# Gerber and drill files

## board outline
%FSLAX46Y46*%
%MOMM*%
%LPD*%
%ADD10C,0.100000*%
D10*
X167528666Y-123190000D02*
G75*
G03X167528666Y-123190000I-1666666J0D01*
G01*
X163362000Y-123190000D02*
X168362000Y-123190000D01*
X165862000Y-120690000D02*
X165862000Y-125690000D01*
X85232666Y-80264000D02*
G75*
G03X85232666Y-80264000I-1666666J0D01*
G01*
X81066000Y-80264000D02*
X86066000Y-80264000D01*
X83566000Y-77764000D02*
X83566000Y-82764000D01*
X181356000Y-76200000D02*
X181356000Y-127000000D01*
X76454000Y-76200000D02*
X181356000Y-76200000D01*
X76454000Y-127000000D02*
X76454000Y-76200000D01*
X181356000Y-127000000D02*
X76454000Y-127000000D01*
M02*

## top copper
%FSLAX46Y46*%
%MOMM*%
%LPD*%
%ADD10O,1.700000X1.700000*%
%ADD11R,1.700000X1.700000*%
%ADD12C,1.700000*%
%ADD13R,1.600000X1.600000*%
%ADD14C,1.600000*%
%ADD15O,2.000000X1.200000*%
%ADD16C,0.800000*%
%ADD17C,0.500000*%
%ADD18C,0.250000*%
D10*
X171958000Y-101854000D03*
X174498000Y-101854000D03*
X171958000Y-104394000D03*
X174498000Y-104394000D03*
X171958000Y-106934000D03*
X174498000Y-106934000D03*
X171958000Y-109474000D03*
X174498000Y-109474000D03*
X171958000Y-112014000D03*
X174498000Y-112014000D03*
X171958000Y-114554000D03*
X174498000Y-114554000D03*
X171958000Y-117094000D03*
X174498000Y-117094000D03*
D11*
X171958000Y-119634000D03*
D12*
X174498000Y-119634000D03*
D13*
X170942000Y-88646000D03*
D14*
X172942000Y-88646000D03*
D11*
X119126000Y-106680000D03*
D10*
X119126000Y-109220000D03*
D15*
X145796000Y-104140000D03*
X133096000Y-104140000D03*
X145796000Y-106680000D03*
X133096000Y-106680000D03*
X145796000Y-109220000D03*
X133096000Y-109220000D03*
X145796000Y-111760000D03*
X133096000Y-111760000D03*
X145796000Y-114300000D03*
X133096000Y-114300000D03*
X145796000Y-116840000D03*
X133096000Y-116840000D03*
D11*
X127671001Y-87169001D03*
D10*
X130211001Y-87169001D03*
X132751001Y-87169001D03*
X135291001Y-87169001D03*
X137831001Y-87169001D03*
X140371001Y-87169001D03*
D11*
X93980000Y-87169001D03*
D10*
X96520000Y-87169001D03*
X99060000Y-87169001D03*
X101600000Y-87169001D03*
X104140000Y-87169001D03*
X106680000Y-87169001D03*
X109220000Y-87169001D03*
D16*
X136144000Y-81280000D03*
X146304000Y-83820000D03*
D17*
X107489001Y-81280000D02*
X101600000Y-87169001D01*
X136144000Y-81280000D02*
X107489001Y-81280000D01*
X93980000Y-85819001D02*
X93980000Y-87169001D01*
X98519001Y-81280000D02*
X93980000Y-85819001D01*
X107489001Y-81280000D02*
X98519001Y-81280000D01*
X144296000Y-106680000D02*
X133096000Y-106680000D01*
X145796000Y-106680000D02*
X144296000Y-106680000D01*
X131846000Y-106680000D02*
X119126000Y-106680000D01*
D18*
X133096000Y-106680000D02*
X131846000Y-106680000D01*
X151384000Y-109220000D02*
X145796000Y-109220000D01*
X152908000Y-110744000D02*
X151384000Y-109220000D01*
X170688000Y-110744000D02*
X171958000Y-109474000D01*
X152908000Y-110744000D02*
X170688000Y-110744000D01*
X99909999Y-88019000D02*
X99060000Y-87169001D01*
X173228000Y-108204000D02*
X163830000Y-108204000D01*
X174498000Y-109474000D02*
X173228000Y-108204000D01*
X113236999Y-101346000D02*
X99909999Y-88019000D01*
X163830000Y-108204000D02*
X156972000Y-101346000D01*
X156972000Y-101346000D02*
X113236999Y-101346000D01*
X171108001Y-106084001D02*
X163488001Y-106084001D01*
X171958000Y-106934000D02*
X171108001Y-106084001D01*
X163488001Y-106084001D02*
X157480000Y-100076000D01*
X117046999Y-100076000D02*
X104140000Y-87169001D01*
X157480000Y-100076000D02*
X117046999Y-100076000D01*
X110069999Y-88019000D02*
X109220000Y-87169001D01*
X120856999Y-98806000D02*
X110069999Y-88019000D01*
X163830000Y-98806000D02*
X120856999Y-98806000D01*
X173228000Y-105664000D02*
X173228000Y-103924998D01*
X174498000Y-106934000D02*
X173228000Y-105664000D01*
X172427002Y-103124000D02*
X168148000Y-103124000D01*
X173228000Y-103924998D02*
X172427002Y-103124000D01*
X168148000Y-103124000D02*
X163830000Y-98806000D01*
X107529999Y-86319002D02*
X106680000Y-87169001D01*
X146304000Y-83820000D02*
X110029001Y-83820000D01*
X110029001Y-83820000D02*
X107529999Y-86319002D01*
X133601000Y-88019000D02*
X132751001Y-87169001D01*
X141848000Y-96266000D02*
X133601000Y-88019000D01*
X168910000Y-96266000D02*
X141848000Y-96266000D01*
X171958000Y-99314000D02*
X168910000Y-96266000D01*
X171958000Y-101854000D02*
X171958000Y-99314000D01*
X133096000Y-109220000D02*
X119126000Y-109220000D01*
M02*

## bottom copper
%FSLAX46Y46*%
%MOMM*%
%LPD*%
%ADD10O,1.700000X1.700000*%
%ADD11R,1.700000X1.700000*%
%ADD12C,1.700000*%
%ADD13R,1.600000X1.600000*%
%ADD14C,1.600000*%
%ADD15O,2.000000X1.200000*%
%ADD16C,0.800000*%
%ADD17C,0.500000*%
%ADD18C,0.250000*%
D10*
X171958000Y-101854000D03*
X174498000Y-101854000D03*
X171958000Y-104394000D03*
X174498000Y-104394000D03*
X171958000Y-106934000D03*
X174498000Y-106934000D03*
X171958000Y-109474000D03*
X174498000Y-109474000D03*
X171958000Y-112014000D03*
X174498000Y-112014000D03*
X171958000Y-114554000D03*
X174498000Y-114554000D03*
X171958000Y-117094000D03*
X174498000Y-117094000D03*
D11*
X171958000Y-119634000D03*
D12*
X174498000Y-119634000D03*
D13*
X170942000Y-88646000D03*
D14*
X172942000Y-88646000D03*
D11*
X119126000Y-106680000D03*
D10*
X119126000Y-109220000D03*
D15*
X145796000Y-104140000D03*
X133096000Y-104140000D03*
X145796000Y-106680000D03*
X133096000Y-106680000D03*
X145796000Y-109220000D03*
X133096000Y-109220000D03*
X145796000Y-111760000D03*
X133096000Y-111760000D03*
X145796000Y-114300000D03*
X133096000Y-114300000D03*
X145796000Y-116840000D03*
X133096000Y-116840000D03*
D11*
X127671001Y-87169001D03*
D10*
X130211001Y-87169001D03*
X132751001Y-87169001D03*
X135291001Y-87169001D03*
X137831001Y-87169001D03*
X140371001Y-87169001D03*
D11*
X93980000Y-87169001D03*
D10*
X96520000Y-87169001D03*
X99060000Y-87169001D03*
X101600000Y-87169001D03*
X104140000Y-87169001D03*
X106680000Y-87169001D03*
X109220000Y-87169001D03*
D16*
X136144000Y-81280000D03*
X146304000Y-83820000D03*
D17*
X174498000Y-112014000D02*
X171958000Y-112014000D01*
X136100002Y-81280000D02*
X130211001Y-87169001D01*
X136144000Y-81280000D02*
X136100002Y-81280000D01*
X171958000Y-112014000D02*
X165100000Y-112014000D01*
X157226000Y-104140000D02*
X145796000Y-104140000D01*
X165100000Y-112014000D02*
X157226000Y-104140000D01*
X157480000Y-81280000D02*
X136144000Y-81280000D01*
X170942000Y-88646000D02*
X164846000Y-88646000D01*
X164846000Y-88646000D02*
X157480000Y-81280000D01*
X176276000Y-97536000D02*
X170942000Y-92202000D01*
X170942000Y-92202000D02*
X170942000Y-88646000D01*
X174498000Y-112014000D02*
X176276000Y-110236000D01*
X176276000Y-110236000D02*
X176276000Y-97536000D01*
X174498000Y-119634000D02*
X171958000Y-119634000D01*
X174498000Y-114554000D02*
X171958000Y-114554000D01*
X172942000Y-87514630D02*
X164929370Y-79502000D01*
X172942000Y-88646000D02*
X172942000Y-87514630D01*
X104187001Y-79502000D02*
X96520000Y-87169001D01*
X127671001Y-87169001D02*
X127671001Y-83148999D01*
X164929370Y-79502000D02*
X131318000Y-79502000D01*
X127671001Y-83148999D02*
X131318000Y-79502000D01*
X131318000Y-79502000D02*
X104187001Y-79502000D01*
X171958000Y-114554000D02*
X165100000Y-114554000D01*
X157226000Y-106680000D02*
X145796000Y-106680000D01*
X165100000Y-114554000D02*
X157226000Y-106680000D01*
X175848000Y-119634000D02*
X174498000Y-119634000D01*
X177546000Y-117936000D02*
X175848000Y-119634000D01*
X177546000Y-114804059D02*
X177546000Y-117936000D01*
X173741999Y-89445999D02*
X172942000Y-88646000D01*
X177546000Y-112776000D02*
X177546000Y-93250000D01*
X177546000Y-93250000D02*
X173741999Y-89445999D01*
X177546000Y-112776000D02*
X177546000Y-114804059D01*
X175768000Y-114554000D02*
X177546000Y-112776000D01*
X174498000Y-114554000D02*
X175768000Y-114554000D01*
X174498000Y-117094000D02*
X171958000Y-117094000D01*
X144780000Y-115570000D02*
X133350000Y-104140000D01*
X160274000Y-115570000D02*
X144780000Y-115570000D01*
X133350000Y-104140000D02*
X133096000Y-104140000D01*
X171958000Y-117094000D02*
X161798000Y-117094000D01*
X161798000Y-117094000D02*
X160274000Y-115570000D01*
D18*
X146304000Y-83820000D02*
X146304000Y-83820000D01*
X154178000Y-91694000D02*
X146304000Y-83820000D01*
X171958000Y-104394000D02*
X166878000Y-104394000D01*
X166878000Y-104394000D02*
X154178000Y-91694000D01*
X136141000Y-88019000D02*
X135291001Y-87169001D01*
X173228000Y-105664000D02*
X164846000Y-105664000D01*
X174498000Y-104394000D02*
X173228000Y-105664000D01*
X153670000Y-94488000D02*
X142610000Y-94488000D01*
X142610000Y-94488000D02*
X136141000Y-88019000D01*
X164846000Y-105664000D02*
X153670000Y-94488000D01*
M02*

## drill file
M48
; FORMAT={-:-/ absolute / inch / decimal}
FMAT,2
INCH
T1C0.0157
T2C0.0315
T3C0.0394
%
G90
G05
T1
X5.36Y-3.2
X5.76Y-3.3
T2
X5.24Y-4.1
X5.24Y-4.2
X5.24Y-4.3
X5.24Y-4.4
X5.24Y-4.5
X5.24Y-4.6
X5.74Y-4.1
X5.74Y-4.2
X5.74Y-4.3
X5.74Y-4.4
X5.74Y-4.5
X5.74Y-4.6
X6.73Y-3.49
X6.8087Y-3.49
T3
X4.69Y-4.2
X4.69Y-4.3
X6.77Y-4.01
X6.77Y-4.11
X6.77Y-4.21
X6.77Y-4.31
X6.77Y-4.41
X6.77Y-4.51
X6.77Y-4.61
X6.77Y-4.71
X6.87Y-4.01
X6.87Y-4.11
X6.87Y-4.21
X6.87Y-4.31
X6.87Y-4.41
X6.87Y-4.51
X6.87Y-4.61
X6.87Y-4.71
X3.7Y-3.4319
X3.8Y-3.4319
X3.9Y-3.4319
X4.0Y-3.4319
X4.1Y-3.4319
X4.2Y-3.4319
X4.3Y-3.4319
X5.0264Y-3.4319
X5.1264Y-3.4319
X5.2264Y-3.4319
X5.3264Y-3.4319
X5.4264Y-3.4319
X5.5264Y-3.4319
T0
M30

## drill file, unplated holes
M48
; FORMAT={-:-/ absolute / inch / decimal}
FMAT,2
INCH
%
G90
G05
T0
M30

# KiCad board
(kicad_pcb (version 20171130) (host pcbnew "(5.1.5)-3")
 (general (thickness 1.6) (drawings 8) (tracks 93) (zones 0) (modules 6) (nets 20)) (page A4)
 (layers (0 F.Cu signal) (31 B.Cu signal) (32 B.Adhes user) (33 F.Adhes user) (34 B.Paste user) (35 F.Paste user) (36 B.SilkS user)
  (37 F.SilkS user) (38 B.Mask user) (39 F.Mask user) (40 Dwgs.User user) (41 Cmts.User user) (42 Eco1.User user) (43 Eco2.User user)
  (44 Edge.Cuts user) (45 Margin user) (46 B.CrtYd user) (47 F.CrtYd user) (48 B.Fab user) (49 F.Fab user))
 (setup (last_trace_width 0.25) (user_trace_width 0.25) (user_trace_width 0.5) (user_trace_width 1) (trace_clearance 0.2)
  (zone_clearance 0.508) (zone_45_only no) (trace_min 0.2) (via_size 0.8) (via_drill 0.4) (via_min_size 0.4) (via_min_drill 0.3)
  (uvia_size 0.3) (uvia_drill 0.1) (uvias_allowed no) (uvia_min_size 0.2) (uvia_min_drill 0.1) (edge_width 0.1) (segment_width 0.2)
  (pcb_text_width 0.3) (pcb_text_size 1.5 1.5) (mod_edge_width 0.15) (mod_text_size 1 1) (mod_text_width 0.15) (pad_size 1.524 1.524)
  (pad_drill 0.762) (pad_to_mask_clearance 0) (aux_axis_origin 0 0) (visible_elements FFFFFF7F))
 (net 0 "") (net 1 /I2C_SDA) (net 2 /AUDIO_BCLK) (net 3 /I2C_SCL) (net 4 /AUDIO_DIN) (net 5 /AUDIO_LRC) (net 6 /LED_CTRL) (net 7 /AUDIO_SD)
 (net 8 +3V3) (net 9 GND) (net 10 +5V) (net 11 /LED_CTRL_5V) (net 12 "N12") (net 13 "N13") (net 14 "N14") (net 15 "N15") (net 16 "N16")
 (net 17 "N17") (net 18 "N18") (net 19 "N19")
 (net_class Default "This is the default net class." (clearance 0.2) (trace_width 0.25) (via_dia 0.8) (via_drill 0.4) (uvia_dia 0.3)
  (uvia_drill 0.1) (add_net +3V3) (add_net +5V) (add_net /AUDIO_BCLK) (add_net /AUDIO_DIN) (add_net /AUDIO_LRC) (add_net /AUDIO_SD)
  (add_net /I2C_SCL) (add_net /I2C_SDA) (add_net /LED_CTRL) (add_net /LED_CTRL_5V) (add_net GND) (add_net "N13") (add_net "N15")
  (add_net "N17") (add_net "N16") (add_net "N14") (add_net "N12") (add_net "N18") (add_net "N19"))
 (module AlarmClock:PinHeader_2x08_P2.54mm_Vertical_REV (layer F.Cu) (at 174.498 119.634 180)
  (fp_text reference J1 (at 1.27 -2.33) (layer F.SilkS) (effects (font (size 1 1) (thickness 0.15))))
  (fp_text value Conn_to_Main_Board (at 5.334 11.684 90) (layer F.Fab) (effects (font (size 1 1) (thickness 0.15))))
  (pad 15 thru_hole oval (at 2.54 17.78 180) (size 1.7 1.7) (drill 1) (layers *.Cu *.Mask) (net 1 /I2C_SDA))
  (pad 16 thru_hole oval (at 0 17.78 180) (size 1.7 1.7) (drill 1) (layers *.Cu *.Mask))
  (pad 13 thru_hole oval (at 2.54 15.24 180) (size 1.7 1.7) (drill 1) (layers *.Cu *.Mask) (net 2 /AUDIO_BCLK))
  (pad 14 thru_hole oval (at 0 15.24 180) (size 1.7 1.7) (drill 1) (layers *.Cu *.Mask) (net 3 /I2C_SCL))
  (pad 11 thru_hole oval (at 2.54 12.7 180) (size 1.7 1.7) (drill 1) (layers *.Cu *.Mask) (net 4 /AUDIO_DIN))
  (pad 12 thru_hole oval (at 0 12.7 180) (size 1.7 1.7) (drill 1) (layers *.Cu *.Mask) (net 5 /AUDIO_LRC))
  (pad 9 thru_hole oval (at 2.54 10.16 180) (size 1.7 1.7) (drill 1) (layers *.Cu *.Mask) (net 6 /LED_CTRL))
  (pad 10 thru_hole oval (at 0 10.16 180) (size 1.7 1.7) (drill 1) (layers *.Cu *.Mask) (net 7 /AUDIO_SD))
  (pad 7 thru_hole oval (at 2.54 7.62 180) (size 1.7 1.7) (drill 1) (layers *.Cu *.Mask) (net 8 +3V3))
  (pad 8 thru_hole oval (at 0 7.62 180) (size 1.7 1.7) (drill 1) (layers *.Cu *.Mask) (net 8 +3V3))
  (pad 5 thru_hole oval (at 2.54 5.08 180) (size 1.7 1.7) (drill 1) (layers *.Cu *.Mask) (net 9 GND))
  (pad 6 thru_hole oval (at 0 5.08 180) (size 1.7 1.7) (drill 1) (layers *.Cu *.Mask) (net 9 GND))
  (pad 3 thru_hole oval (at 2.54 2.54 180) (size 1.7 1.7) (drill 1) (layers *.Cu *.Mask) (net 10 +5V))
  (pad 4 thru_hole oval (at 0 2.54 180) (size 1.7 1.7) (drill 1) (layers *.Cu *.Mask) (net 10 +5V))
  (pad 1 thru_hole rect (at 2.54 0 180) (size 1.7 1.7) (drill 1) (layers *.Cu *.Mask) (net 9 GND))
  (pad 2 thru_hole circle (at 0 0 180) (size 1.7 1.7) (drill 1) (layers *.Cu *.Mask) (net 9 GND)))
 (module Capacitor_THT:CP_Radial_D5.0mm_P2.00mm (layer F.Cu) (at 170.942 88.646)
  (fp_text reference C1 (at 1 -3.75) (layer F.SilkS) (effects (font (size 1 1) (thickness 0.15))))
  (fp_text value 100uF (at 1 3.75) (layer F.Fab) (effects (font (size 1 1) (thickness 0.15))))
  (pad 1 thru_hole rect (at 0 0) (size 1.6 1.6) (drill 0.8) (layers *.Cu *.Mask) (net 8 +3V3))
  (pad 2 thru_hole circle (at 2 0) (size 1.6 1.6) (drill 0.8) (layers *.Cu *.Mask) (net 9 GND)))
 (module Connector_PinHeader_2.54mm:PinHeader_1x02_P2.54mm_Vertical (layer F.Cu) (at 119.126 106.68)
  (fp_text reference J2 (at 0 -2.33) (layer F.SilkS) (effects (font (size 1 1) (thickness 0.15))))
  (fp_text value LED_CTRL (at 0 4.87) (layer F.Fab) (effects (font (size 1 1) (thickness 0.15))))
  (pad 1 thru_hole rect (at 0 0) (size 1.7 1.7) (drill 1) (layers *.Cu *.Mask) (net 9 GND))
  (pad 2 thru_hole oval (at 0 2.54) (size 1.7 1.7) (drill 1) (layers *.Cu *.Mask) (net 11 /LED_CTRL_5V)))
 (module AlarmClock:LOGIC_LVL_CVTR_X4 (layer F.Cu) (at 131.826 118.11)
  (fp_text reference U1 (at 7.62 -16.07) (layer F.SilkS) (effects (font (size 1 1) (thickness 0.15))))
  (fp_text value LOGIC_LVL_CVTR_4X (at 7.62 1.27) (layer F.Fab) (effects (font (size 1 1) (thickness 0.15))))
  (pad 12 thru_hole oval (at 13.97 -13.97 270) (size 1.2 2) (drill 0.8) (layers *.Cu *.Mask) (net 8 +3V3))
  (pad 1 thru_hole oval (at 1.27 -13.97 270) (size 1.2 2) (drill 0.8) (layers *.Cu *.Mask) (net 10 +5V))
  (pad 11 thru_hole oval (at 13.97 -11.43 270) (size 1.2 2) (drill 0.8) (layers *.Cu *.Mask) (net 9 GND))
  (pad 2 thru_hole oval (at 1.27 -11.43 270) (size 1.2 2) (drill 0.8) (layers *.Cu *.Mask) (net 9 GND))
  (pad 10 thru_hole oval (at 13.97 -8.89 270) (size 1.2 2) (drill 0.8) (layers *.Cu *.Mask) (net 6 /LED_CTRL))
  (pad 3 thru_hole oval (at 1.27 -8.89 270) (size 1.2 2) (drill 0.8) (layers *.Cu *.Mask) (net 11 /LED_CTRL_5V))
  (pad 9 thru_hole oval (at 13.97 -6.35 270) (size 1.2 2) (drill 0.8) (layers *.Cu *.Mask) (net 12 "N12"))
  (pad 4 thru_hole oval (at 1.27 -6.35 270) (size 1.2 2) (drill 0.8) (layers *.Cu *.Mask) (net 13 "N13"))
  (pad 8 thru_hole oval (at 13.97 -3.81 270) (size 1.2 2) (drill 0.8) (layers *.Cu *.Mask) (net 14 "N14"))
  (pad 5 thru_hole oval (at 1.27 -3.81 270) (size 1.2 2) (drill 0.8) (layers *.Cu *.Mask) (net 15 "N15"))
  (pad 7 thru_hole oval (at 13.97 -1.27 270) (size 1.2 2) (drill 0.8) (layers *.Cu *.Mask) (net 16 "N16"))
  (pad 6 thru_hole oval (at 1.27 -1.27 270) (size 1.2 2) (drill 0.8) (layers *.Cu *.Mask) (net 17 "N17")))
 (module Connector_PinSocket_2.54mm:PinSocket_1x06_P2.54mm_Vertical (layer F.Cu) (at 127.671001 87.169001 90)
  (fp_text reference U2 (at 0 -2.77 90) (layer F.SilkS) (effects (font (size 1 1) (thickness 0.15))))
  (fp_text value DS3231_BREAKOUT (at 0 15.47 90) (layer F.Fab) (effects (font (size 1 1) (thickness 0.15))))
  (pad 1 thru_hole rect (at 0 0 90) (size 1.7 1.7) (drill 1) (layers *.Cu *.Mask) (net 9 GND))
  (pad 2 thru_hole oval (at 0 2.54 90) (size 1.7 1.7) (drill 1) (layers *.Cu *.Mask) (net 8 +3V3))
  (pad 3 thru_hole oval (at 0 5.08 90) (size 1.7 1.7) (drill 1) (layers *.Cu *.Mask) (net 1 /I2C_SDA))
  (pad 4 thru_hole oval (at 0 7.62 90) (size 1.7 1.7) (drill 1) (layers *.Cu *.Mask) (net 3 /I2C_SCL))
  (pad 5 thru_hole oval (at 0 10.16 90) (size 1.7 1.7) (drill 1) (layers *.Cu *.Mask) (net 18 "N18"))
  (pad 6 thru_hole oval (at 0 12.7 90) (size 1.7 1.7) (drill 1) (layers *.Cu *.Mask) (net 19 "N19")))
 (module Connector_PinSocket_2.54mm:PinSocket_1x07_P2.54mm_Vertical (layer F.Cu) (at 93.98 87.169001 90)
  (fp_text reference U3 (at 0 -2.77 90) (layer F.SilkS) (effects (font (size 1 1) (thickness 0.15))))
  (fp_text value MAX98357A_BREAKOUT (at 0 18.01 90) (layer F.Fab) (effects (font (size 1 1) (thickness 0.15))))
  (pad 1 thru_hole rect (at 0 0 90) (size 1.7 1.7) (drill 1) (layers *.Cu *.Mask) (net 8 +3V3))
  (pad 2 thru_hole oval (at 0 2.54 90) (size 1.7 1.7) (drill 1) (layers *.Cu *.Mask) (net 9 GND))
  (pad 3 thru_hole oval (at 0 5.08 90) (size 1.7 1.7) (drill 1) (layers *.Cu *.Mask) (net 7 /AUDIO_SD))
  (pad 4 thru_hole oval (at 0 7.62 90) (size 1.7 1.7) (drill 1) (layers *.Cu *.Mask) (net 8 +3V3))
  (pad 5 thru_hole oval (at 0 10.16 90) (size 1.7 1.7) (drill 1) (layers *.Cu *.Mask) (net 4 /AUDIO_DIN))
  (pad 6 thru_hole oval (at 0 12.7 90) (size 1.7 1.7) (drill 1) (layers *.Cu *.Mask) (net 2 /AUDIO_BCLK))
  (pad 7 thru_hole oval (at 0 15.24 90) (size 1.7 1.7) (drill 1) (layers *.Cu *.Mask) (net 5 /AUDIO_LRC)))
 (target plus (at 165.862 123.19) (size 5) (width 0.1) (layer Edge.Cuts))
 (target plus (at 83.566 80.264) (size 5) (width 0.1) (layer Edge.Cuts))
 (gr_line (start 181.356 76.2) (end 181.356 127) (layer Edge.Cuts) (width 0.1))
 (gr_line (start 76.454 76.2) (end 181.356 76.2) (layer Edge.Cuts) (width 0.1))
 (gr_line (start 76.454 127) (end 76.454 76.2) (layer Edge.Cuts) (width 0.1))
 (gr_line (start 181.356 127) (end 76.454 127) (layer Edge.Cuts) (width 0.1))
 (segment (start 174.498 112.014) (end 171.958 112.014) (width 0.5) (layer B.Cu) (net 8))
 (segment (start 136.100002 81.28) (end 130.211001 87.169001) (width 0.5) (layer B.Cu) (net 8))
 (segment (start 136.144 81.28) (end 136.100002 81.28) (width 0.5) (layer B.Cu) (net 8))
 (via (at 136.144 81.28) (size 0.8) (drill 0.4) (layers F.Cu B.Cu) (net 8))
 (segment (start 107.489001 81.28) (end 101.6 87.169001) (width 0.5) (layer F.Cu) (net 8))
 (segment (start 136.144 81.28) (end 107.489001 81.28) (width 0.5) (layer F.Cu) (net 8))
 (segment (start 93.98 85.819001) (end 93.98 87.169001) (width 0.5) (layer F.Cu) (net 8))
 (segment (start 98.519001 81.28) (end 93.98 85.819001) (width 0.5) (layer F.Cu) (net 8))
 (segment (start 107.489001 81.28) (end 98.519001 81.28) (width 0.5) (layer F.Cu) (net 8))
 (segment (start 171.958 112.014) (end 165.1 112.014) (width 0.5) (layer B.Cu) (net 8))
 (segment (start 157.226 104.14) (end 145.796 104.14) (width 0.5) (layer B.Cu) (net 8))
 (segment (start 165.1 112.014) (end 157.226 104.14) (width 0.5) (layer B.Cu) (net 8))
 (segment (start 157.48 81.28) (end 136.144 81.28) (width 0.5) (layer B.Cu) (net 8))
 (segment (start 170.942 88.646) (end 164.846 88.646) (width 0.5) (layer B.Cu) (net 8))
 (segment (start 164.846 88.646) (end 157.48 81.28) (width 0.5) (layer B.Cu) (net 8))
 (segment (start 176.276 97.536) (end 170.942 92.202) (width 0.5) (layer B.Cu) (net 8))
 (segment (start 170.942 92.202) (end 170.942 88.646) (width 0.5) (layer B.Cu) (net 8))
 (segment (start 174.498 112.014) (end 176.276 110.236) (width 0.5) (layer B.Cu) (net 8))
 (segment (start 176.276 110.236) (end 176.276 97.536) (width 0.5) (layer B.Cu) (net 8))
 (segment (start 174.498 119.634) (end 171.958 119.634) (width 0.5) (layer B.Cu) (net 9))
 (segment (start 174.498 114.554) (end 171.958 114.554) (width 0.5) (layer B.Cu) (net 9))
 (segment (start 172.942 87.51463) (end 164.92937 79.502) (width 0.5) (layer B.Cu) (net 9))
 (segment (start 172.942 88.646) (end 172.942 87.51463) (width 0.5) (layer B.Cu) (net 9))
 (segment (start 104.187001 79.502) (end 96.52 87.169001) (width 0.5) (layer B.Cu) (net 9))
 (segment (start 127.671001 87.169001) (end 127.671001 83.148999) (width 0.5) (layer B.Cu) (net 9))
 (segment (start 164.92937 79.502) (end 131.318 79.502) (width 0.5) (layer B.Cu) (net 9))
 (segment (start 127.671001 83.148999) (end 131.318 79.502) (width 0.5) (layer B.Cu) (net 9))
 (segment (start 131.318 79.502) (end 104.187001 79.502) (width 0.5) (layer B.Cu) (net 9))
 (segment (start 171.958 114.554) (end 165.1 114.554) (width 0.5) (layer B.Cu) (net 9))
 (segment (start 157.226 106.68) (end 145.796 106.68) (width 0.5) (layer B.Cu) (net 9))
 (segment (start 165.1 114.554) (end 157.226 106.68) (width 0.5) (layer B.Cu) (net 9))
 (segment (start 144.296 106.68) (end 133.096 106.68) (width 0.5) (layer F.Cu) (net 9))
 (segment (start 145.796 106.68) (end 144.296 106.68) (width 0.5) (layer F.Cu) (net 9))
 (segment (start 131.846 106.68) (end 119.126 106.68) (width 0.5) (layer F.Cu) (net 9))
 (segment (start 133.096 106.68) (end 131.846 106.68) (width 0.25) (layer F.Cu) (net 9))
 (segment (start 175.848 119.634) (end 174.498 119.634) (width 0.5) (layer B.Cu) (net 9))
 (segment (start 177.546 117.936) (end 175.848 119.634) (width 0.5) (layer B.Cu) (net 9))
 (segment (start 177.546 114.804059) (end 177.546 117.936) (width 0.5) (layer B.Cu) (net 9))
 (segment (start 173.741999 89.445999) (end 172.942 88.646) (width 0.5) (layer B.Cu) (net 9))
 (segment (start 177.546 112.776) (end 177.546 93.25) (width 0.5) (layer B.Cu) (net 9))
 (segment (start 177.546 93.25) (end 173.741999 89.445999) (width 0.5) (layer B.Cu) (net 9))
 (segment (start 177.546 112.776) (end 177.546 114.804059) (width 0.5) (layer B.Cu) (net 9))
 (segment (start 175.768 114.554) (end 177.546 112.776) (width 0.5) (layer B.Cu) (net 9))
 (segment (start 174.498 114.554) (end 175.768 114.554) (width 0.5) (layer B.Cu) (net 9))
 (segment (start 174.498 117.094) (end 171.958 117.094) (width 0.5) (layer B.Cu) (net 10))
 (segment (start 144.78 115.57) (end 133.35 104.14) (width 0.5) (layer B.Cu) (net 10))
 (segment (start 160.274 115.57) (end 144.78 115.57) (width 0.5) (layer B.Cu) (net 10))
 (segment (start 133.35 104.14) (end 133.096 104.14) (width 0.5) (layer B.Cu) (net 10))
 (segment (start 171.958 117.094) (end 161.798 117.094) (width 0.5) (layer B.Cu) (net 10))
 (segment (start 161.798 117.094) (end 160.274 115.57) (width 0.5) (layer B.Cu) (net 10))
 (segment (start 151.384 109.22) (end 145.796 109.22) (width 0.25) (layer F.Cu) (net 6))
 (segment (start 152.908 110.744) (end 151.384 109.22) (width 0.25) (layer F.Cu) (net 6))
 (segment (start 170.688 110.744) (end 171.958 109.474) (width 0.25) (layer F.Cu) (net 6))
 (segment (start 152.908 110.744) (end 170.688 110.744) (width 0.25) (layer F.Cu) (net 6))
 (segment (start 99.909999 88.019) (end 99.06 87.169001) (width 0.25) (layer F.Cu) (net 7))
 (segment (start 173.228 108.204) (end 163.83 108.204) (width 0.25) (layer F.Cu) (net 7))
 (segment (start 174.498 109.474) (end 173.228 108.204) (width 0.25) (layer F.Cu) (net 7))
 (segment (start 113.236999 101.346) (end 99.909999 88.019) (width 0.25) (layer F.Cu) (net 7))
 (segment (start 163.83 108.204) (end 156.972 101.346) (width 0.25) (layer F.Cu) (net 7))
 (segment (start 156.972 101.346) (end 113.236999 101.346) (width 0.25) (layer F.Cu) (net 7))
 (segment (start 171.108001 106.084001) (end 163.488001 106.084001) (width 0.25) (layer F.Cu) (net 4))
 (segment (start 171.958 106.934) (end 171.108001 106.084001) (width 0.25) (layer F.Cu) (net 4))
 (segment (start 163.488001 106.084001) (end 157.48 100.076) (width 0.25) (layer F.Cu) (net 4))
 (segment (start 117.046999 100.076) (end 104.14 87.169001) (width 0.25) (layer F.Cu) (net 4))
 (segment (start 157.48 100.076) (end 117.046999 100.076) (width 0.25) (layer F.Cu) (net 4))
 (segment (start 110.069999 88.019) (end 109.22 87.169001) (width 0.25) (layer F.Cu) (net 5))
 (segment (start 120.856999 98.806) (end 110.069999 88.019) (width 0.25) (layer F.Cu) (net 5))
 (segment (start 163.83 98.806) (end 120.856999 98.806) (width 0.25) (layer F.Cu) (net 5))
 (segment (start 173.228 105.664) (end 173.228 103.924998) (width 0.25) (layer F.Cu) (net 5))
 (segment (start 174.498 106.934) (end 173.228 105.664) (width 0.25) (layer F.Cu) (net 5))
 (segment (start 172.427002 103.124) (end 168.148 103.124) (width 0.25) (layer F.Cu) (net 5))
 (segment (start 173.228 103.924998) (end 172.427002 103.124) (width 0.25) (layer F.Cu) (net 5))
 (segment (start 168.148 103.124) (end 163.83 98.806) (width 0.25) (layer F.Cu) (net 5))
 (segment (start 146.304 83.82) (end 146.304 83.82) (width 0.25) (layer B.Cu) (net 2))
 (via (at 146.304 83.82) (size 0.8) (drill 0.4) (layers F.Cu B.Cu) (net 2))
 (segment (start 107.529999 86.319002) (end 106.68 87.169001) (width 0.25) (layer F.Cu) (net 2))
 (segment (start 146.304 83.82) (end 110.029001 83.82) (width 0.25) (layer F.Cu) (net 2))
 (segment (start 110.029001 83.82) (end 107.529999 86.319002) (width 0.25) (layer F.Cu) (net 2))
 (segment (start 154.178 91.694) (end 146.304 83.82) (width 0.25) (layer B.Cu) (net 2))
 (segment (start 171.958 104.394) (end 166.878 104.394) (width 0.25) (layer B.Cu) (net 2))
 (segment (start 166.878 104.394) (end 154.178 91.694) (width 0.25) (layer B.Cu) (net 2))
 (segment (start 136.141 88.019) (end 135.291001 87.169001) (width 0.25) (layer B.Cu) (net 3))
 (segment (start 173.228 105.664) (end 164.846 105.664) (width 0.25) (layer B.Cu) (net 3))
 (segment (start 174.498 104.394) (end 173.228 105.664) (width 0.25) (layer B.Cu) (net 3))
 (segment (start 153.67 94.488) (end 142.61 94.488) (width 0.25) (layer B.Cu) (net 3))
 (segment (start 142.61 94.488) (end 136.141 88.019) (width 0.25) (layer B.Cu) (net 3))
 (segment (start 164.846 105.664) (end 153.67 94.488) (width 0.25) (layer B.Cu) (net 3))
 (segment (start 133.601 88.019) (end 132.751001 87.169001) (width 0.25) (layer F.Cu) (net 1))
 (segment (start 141.848 96.266) (end 133.601 88.019) (width 0.25) (layer F.Cu) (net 1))
 (segment (start 168.91 96.266) (end 141.848 96.266) (width 0.25) (layer F.Cu) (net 1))
 (segment (start 171.958 99.314) (end 168.91 96.266) (width 0.25) (layer F.Cu) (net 1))
 (segment (start 171.958 101.854) (end 171.958 99.314) (width 0.25) (layer F.Cu) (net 1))
 (segment (start 133.096 109.22) (end 119.126 109.22) (width 0.25) (layer F.Cu) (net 11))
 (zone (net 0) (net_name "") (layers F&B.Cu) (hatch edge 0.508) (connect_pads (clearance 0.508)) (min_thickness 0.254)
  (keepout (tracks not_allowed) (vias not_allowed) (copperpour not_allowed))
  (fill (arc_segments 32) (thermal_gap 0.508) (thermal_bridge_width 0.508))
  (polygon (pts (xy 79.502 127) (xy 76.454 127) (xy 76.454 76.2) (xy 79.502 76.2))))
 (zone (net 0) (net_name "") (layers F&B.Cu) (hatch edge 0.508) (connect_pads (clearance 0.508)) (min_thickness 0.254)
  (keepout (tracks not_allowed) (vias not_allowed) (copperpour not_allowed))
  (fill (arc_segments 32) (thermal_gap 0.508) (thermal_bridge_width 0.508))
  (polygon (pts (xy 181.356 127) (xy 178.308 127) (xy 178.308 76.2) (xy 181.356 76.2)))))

